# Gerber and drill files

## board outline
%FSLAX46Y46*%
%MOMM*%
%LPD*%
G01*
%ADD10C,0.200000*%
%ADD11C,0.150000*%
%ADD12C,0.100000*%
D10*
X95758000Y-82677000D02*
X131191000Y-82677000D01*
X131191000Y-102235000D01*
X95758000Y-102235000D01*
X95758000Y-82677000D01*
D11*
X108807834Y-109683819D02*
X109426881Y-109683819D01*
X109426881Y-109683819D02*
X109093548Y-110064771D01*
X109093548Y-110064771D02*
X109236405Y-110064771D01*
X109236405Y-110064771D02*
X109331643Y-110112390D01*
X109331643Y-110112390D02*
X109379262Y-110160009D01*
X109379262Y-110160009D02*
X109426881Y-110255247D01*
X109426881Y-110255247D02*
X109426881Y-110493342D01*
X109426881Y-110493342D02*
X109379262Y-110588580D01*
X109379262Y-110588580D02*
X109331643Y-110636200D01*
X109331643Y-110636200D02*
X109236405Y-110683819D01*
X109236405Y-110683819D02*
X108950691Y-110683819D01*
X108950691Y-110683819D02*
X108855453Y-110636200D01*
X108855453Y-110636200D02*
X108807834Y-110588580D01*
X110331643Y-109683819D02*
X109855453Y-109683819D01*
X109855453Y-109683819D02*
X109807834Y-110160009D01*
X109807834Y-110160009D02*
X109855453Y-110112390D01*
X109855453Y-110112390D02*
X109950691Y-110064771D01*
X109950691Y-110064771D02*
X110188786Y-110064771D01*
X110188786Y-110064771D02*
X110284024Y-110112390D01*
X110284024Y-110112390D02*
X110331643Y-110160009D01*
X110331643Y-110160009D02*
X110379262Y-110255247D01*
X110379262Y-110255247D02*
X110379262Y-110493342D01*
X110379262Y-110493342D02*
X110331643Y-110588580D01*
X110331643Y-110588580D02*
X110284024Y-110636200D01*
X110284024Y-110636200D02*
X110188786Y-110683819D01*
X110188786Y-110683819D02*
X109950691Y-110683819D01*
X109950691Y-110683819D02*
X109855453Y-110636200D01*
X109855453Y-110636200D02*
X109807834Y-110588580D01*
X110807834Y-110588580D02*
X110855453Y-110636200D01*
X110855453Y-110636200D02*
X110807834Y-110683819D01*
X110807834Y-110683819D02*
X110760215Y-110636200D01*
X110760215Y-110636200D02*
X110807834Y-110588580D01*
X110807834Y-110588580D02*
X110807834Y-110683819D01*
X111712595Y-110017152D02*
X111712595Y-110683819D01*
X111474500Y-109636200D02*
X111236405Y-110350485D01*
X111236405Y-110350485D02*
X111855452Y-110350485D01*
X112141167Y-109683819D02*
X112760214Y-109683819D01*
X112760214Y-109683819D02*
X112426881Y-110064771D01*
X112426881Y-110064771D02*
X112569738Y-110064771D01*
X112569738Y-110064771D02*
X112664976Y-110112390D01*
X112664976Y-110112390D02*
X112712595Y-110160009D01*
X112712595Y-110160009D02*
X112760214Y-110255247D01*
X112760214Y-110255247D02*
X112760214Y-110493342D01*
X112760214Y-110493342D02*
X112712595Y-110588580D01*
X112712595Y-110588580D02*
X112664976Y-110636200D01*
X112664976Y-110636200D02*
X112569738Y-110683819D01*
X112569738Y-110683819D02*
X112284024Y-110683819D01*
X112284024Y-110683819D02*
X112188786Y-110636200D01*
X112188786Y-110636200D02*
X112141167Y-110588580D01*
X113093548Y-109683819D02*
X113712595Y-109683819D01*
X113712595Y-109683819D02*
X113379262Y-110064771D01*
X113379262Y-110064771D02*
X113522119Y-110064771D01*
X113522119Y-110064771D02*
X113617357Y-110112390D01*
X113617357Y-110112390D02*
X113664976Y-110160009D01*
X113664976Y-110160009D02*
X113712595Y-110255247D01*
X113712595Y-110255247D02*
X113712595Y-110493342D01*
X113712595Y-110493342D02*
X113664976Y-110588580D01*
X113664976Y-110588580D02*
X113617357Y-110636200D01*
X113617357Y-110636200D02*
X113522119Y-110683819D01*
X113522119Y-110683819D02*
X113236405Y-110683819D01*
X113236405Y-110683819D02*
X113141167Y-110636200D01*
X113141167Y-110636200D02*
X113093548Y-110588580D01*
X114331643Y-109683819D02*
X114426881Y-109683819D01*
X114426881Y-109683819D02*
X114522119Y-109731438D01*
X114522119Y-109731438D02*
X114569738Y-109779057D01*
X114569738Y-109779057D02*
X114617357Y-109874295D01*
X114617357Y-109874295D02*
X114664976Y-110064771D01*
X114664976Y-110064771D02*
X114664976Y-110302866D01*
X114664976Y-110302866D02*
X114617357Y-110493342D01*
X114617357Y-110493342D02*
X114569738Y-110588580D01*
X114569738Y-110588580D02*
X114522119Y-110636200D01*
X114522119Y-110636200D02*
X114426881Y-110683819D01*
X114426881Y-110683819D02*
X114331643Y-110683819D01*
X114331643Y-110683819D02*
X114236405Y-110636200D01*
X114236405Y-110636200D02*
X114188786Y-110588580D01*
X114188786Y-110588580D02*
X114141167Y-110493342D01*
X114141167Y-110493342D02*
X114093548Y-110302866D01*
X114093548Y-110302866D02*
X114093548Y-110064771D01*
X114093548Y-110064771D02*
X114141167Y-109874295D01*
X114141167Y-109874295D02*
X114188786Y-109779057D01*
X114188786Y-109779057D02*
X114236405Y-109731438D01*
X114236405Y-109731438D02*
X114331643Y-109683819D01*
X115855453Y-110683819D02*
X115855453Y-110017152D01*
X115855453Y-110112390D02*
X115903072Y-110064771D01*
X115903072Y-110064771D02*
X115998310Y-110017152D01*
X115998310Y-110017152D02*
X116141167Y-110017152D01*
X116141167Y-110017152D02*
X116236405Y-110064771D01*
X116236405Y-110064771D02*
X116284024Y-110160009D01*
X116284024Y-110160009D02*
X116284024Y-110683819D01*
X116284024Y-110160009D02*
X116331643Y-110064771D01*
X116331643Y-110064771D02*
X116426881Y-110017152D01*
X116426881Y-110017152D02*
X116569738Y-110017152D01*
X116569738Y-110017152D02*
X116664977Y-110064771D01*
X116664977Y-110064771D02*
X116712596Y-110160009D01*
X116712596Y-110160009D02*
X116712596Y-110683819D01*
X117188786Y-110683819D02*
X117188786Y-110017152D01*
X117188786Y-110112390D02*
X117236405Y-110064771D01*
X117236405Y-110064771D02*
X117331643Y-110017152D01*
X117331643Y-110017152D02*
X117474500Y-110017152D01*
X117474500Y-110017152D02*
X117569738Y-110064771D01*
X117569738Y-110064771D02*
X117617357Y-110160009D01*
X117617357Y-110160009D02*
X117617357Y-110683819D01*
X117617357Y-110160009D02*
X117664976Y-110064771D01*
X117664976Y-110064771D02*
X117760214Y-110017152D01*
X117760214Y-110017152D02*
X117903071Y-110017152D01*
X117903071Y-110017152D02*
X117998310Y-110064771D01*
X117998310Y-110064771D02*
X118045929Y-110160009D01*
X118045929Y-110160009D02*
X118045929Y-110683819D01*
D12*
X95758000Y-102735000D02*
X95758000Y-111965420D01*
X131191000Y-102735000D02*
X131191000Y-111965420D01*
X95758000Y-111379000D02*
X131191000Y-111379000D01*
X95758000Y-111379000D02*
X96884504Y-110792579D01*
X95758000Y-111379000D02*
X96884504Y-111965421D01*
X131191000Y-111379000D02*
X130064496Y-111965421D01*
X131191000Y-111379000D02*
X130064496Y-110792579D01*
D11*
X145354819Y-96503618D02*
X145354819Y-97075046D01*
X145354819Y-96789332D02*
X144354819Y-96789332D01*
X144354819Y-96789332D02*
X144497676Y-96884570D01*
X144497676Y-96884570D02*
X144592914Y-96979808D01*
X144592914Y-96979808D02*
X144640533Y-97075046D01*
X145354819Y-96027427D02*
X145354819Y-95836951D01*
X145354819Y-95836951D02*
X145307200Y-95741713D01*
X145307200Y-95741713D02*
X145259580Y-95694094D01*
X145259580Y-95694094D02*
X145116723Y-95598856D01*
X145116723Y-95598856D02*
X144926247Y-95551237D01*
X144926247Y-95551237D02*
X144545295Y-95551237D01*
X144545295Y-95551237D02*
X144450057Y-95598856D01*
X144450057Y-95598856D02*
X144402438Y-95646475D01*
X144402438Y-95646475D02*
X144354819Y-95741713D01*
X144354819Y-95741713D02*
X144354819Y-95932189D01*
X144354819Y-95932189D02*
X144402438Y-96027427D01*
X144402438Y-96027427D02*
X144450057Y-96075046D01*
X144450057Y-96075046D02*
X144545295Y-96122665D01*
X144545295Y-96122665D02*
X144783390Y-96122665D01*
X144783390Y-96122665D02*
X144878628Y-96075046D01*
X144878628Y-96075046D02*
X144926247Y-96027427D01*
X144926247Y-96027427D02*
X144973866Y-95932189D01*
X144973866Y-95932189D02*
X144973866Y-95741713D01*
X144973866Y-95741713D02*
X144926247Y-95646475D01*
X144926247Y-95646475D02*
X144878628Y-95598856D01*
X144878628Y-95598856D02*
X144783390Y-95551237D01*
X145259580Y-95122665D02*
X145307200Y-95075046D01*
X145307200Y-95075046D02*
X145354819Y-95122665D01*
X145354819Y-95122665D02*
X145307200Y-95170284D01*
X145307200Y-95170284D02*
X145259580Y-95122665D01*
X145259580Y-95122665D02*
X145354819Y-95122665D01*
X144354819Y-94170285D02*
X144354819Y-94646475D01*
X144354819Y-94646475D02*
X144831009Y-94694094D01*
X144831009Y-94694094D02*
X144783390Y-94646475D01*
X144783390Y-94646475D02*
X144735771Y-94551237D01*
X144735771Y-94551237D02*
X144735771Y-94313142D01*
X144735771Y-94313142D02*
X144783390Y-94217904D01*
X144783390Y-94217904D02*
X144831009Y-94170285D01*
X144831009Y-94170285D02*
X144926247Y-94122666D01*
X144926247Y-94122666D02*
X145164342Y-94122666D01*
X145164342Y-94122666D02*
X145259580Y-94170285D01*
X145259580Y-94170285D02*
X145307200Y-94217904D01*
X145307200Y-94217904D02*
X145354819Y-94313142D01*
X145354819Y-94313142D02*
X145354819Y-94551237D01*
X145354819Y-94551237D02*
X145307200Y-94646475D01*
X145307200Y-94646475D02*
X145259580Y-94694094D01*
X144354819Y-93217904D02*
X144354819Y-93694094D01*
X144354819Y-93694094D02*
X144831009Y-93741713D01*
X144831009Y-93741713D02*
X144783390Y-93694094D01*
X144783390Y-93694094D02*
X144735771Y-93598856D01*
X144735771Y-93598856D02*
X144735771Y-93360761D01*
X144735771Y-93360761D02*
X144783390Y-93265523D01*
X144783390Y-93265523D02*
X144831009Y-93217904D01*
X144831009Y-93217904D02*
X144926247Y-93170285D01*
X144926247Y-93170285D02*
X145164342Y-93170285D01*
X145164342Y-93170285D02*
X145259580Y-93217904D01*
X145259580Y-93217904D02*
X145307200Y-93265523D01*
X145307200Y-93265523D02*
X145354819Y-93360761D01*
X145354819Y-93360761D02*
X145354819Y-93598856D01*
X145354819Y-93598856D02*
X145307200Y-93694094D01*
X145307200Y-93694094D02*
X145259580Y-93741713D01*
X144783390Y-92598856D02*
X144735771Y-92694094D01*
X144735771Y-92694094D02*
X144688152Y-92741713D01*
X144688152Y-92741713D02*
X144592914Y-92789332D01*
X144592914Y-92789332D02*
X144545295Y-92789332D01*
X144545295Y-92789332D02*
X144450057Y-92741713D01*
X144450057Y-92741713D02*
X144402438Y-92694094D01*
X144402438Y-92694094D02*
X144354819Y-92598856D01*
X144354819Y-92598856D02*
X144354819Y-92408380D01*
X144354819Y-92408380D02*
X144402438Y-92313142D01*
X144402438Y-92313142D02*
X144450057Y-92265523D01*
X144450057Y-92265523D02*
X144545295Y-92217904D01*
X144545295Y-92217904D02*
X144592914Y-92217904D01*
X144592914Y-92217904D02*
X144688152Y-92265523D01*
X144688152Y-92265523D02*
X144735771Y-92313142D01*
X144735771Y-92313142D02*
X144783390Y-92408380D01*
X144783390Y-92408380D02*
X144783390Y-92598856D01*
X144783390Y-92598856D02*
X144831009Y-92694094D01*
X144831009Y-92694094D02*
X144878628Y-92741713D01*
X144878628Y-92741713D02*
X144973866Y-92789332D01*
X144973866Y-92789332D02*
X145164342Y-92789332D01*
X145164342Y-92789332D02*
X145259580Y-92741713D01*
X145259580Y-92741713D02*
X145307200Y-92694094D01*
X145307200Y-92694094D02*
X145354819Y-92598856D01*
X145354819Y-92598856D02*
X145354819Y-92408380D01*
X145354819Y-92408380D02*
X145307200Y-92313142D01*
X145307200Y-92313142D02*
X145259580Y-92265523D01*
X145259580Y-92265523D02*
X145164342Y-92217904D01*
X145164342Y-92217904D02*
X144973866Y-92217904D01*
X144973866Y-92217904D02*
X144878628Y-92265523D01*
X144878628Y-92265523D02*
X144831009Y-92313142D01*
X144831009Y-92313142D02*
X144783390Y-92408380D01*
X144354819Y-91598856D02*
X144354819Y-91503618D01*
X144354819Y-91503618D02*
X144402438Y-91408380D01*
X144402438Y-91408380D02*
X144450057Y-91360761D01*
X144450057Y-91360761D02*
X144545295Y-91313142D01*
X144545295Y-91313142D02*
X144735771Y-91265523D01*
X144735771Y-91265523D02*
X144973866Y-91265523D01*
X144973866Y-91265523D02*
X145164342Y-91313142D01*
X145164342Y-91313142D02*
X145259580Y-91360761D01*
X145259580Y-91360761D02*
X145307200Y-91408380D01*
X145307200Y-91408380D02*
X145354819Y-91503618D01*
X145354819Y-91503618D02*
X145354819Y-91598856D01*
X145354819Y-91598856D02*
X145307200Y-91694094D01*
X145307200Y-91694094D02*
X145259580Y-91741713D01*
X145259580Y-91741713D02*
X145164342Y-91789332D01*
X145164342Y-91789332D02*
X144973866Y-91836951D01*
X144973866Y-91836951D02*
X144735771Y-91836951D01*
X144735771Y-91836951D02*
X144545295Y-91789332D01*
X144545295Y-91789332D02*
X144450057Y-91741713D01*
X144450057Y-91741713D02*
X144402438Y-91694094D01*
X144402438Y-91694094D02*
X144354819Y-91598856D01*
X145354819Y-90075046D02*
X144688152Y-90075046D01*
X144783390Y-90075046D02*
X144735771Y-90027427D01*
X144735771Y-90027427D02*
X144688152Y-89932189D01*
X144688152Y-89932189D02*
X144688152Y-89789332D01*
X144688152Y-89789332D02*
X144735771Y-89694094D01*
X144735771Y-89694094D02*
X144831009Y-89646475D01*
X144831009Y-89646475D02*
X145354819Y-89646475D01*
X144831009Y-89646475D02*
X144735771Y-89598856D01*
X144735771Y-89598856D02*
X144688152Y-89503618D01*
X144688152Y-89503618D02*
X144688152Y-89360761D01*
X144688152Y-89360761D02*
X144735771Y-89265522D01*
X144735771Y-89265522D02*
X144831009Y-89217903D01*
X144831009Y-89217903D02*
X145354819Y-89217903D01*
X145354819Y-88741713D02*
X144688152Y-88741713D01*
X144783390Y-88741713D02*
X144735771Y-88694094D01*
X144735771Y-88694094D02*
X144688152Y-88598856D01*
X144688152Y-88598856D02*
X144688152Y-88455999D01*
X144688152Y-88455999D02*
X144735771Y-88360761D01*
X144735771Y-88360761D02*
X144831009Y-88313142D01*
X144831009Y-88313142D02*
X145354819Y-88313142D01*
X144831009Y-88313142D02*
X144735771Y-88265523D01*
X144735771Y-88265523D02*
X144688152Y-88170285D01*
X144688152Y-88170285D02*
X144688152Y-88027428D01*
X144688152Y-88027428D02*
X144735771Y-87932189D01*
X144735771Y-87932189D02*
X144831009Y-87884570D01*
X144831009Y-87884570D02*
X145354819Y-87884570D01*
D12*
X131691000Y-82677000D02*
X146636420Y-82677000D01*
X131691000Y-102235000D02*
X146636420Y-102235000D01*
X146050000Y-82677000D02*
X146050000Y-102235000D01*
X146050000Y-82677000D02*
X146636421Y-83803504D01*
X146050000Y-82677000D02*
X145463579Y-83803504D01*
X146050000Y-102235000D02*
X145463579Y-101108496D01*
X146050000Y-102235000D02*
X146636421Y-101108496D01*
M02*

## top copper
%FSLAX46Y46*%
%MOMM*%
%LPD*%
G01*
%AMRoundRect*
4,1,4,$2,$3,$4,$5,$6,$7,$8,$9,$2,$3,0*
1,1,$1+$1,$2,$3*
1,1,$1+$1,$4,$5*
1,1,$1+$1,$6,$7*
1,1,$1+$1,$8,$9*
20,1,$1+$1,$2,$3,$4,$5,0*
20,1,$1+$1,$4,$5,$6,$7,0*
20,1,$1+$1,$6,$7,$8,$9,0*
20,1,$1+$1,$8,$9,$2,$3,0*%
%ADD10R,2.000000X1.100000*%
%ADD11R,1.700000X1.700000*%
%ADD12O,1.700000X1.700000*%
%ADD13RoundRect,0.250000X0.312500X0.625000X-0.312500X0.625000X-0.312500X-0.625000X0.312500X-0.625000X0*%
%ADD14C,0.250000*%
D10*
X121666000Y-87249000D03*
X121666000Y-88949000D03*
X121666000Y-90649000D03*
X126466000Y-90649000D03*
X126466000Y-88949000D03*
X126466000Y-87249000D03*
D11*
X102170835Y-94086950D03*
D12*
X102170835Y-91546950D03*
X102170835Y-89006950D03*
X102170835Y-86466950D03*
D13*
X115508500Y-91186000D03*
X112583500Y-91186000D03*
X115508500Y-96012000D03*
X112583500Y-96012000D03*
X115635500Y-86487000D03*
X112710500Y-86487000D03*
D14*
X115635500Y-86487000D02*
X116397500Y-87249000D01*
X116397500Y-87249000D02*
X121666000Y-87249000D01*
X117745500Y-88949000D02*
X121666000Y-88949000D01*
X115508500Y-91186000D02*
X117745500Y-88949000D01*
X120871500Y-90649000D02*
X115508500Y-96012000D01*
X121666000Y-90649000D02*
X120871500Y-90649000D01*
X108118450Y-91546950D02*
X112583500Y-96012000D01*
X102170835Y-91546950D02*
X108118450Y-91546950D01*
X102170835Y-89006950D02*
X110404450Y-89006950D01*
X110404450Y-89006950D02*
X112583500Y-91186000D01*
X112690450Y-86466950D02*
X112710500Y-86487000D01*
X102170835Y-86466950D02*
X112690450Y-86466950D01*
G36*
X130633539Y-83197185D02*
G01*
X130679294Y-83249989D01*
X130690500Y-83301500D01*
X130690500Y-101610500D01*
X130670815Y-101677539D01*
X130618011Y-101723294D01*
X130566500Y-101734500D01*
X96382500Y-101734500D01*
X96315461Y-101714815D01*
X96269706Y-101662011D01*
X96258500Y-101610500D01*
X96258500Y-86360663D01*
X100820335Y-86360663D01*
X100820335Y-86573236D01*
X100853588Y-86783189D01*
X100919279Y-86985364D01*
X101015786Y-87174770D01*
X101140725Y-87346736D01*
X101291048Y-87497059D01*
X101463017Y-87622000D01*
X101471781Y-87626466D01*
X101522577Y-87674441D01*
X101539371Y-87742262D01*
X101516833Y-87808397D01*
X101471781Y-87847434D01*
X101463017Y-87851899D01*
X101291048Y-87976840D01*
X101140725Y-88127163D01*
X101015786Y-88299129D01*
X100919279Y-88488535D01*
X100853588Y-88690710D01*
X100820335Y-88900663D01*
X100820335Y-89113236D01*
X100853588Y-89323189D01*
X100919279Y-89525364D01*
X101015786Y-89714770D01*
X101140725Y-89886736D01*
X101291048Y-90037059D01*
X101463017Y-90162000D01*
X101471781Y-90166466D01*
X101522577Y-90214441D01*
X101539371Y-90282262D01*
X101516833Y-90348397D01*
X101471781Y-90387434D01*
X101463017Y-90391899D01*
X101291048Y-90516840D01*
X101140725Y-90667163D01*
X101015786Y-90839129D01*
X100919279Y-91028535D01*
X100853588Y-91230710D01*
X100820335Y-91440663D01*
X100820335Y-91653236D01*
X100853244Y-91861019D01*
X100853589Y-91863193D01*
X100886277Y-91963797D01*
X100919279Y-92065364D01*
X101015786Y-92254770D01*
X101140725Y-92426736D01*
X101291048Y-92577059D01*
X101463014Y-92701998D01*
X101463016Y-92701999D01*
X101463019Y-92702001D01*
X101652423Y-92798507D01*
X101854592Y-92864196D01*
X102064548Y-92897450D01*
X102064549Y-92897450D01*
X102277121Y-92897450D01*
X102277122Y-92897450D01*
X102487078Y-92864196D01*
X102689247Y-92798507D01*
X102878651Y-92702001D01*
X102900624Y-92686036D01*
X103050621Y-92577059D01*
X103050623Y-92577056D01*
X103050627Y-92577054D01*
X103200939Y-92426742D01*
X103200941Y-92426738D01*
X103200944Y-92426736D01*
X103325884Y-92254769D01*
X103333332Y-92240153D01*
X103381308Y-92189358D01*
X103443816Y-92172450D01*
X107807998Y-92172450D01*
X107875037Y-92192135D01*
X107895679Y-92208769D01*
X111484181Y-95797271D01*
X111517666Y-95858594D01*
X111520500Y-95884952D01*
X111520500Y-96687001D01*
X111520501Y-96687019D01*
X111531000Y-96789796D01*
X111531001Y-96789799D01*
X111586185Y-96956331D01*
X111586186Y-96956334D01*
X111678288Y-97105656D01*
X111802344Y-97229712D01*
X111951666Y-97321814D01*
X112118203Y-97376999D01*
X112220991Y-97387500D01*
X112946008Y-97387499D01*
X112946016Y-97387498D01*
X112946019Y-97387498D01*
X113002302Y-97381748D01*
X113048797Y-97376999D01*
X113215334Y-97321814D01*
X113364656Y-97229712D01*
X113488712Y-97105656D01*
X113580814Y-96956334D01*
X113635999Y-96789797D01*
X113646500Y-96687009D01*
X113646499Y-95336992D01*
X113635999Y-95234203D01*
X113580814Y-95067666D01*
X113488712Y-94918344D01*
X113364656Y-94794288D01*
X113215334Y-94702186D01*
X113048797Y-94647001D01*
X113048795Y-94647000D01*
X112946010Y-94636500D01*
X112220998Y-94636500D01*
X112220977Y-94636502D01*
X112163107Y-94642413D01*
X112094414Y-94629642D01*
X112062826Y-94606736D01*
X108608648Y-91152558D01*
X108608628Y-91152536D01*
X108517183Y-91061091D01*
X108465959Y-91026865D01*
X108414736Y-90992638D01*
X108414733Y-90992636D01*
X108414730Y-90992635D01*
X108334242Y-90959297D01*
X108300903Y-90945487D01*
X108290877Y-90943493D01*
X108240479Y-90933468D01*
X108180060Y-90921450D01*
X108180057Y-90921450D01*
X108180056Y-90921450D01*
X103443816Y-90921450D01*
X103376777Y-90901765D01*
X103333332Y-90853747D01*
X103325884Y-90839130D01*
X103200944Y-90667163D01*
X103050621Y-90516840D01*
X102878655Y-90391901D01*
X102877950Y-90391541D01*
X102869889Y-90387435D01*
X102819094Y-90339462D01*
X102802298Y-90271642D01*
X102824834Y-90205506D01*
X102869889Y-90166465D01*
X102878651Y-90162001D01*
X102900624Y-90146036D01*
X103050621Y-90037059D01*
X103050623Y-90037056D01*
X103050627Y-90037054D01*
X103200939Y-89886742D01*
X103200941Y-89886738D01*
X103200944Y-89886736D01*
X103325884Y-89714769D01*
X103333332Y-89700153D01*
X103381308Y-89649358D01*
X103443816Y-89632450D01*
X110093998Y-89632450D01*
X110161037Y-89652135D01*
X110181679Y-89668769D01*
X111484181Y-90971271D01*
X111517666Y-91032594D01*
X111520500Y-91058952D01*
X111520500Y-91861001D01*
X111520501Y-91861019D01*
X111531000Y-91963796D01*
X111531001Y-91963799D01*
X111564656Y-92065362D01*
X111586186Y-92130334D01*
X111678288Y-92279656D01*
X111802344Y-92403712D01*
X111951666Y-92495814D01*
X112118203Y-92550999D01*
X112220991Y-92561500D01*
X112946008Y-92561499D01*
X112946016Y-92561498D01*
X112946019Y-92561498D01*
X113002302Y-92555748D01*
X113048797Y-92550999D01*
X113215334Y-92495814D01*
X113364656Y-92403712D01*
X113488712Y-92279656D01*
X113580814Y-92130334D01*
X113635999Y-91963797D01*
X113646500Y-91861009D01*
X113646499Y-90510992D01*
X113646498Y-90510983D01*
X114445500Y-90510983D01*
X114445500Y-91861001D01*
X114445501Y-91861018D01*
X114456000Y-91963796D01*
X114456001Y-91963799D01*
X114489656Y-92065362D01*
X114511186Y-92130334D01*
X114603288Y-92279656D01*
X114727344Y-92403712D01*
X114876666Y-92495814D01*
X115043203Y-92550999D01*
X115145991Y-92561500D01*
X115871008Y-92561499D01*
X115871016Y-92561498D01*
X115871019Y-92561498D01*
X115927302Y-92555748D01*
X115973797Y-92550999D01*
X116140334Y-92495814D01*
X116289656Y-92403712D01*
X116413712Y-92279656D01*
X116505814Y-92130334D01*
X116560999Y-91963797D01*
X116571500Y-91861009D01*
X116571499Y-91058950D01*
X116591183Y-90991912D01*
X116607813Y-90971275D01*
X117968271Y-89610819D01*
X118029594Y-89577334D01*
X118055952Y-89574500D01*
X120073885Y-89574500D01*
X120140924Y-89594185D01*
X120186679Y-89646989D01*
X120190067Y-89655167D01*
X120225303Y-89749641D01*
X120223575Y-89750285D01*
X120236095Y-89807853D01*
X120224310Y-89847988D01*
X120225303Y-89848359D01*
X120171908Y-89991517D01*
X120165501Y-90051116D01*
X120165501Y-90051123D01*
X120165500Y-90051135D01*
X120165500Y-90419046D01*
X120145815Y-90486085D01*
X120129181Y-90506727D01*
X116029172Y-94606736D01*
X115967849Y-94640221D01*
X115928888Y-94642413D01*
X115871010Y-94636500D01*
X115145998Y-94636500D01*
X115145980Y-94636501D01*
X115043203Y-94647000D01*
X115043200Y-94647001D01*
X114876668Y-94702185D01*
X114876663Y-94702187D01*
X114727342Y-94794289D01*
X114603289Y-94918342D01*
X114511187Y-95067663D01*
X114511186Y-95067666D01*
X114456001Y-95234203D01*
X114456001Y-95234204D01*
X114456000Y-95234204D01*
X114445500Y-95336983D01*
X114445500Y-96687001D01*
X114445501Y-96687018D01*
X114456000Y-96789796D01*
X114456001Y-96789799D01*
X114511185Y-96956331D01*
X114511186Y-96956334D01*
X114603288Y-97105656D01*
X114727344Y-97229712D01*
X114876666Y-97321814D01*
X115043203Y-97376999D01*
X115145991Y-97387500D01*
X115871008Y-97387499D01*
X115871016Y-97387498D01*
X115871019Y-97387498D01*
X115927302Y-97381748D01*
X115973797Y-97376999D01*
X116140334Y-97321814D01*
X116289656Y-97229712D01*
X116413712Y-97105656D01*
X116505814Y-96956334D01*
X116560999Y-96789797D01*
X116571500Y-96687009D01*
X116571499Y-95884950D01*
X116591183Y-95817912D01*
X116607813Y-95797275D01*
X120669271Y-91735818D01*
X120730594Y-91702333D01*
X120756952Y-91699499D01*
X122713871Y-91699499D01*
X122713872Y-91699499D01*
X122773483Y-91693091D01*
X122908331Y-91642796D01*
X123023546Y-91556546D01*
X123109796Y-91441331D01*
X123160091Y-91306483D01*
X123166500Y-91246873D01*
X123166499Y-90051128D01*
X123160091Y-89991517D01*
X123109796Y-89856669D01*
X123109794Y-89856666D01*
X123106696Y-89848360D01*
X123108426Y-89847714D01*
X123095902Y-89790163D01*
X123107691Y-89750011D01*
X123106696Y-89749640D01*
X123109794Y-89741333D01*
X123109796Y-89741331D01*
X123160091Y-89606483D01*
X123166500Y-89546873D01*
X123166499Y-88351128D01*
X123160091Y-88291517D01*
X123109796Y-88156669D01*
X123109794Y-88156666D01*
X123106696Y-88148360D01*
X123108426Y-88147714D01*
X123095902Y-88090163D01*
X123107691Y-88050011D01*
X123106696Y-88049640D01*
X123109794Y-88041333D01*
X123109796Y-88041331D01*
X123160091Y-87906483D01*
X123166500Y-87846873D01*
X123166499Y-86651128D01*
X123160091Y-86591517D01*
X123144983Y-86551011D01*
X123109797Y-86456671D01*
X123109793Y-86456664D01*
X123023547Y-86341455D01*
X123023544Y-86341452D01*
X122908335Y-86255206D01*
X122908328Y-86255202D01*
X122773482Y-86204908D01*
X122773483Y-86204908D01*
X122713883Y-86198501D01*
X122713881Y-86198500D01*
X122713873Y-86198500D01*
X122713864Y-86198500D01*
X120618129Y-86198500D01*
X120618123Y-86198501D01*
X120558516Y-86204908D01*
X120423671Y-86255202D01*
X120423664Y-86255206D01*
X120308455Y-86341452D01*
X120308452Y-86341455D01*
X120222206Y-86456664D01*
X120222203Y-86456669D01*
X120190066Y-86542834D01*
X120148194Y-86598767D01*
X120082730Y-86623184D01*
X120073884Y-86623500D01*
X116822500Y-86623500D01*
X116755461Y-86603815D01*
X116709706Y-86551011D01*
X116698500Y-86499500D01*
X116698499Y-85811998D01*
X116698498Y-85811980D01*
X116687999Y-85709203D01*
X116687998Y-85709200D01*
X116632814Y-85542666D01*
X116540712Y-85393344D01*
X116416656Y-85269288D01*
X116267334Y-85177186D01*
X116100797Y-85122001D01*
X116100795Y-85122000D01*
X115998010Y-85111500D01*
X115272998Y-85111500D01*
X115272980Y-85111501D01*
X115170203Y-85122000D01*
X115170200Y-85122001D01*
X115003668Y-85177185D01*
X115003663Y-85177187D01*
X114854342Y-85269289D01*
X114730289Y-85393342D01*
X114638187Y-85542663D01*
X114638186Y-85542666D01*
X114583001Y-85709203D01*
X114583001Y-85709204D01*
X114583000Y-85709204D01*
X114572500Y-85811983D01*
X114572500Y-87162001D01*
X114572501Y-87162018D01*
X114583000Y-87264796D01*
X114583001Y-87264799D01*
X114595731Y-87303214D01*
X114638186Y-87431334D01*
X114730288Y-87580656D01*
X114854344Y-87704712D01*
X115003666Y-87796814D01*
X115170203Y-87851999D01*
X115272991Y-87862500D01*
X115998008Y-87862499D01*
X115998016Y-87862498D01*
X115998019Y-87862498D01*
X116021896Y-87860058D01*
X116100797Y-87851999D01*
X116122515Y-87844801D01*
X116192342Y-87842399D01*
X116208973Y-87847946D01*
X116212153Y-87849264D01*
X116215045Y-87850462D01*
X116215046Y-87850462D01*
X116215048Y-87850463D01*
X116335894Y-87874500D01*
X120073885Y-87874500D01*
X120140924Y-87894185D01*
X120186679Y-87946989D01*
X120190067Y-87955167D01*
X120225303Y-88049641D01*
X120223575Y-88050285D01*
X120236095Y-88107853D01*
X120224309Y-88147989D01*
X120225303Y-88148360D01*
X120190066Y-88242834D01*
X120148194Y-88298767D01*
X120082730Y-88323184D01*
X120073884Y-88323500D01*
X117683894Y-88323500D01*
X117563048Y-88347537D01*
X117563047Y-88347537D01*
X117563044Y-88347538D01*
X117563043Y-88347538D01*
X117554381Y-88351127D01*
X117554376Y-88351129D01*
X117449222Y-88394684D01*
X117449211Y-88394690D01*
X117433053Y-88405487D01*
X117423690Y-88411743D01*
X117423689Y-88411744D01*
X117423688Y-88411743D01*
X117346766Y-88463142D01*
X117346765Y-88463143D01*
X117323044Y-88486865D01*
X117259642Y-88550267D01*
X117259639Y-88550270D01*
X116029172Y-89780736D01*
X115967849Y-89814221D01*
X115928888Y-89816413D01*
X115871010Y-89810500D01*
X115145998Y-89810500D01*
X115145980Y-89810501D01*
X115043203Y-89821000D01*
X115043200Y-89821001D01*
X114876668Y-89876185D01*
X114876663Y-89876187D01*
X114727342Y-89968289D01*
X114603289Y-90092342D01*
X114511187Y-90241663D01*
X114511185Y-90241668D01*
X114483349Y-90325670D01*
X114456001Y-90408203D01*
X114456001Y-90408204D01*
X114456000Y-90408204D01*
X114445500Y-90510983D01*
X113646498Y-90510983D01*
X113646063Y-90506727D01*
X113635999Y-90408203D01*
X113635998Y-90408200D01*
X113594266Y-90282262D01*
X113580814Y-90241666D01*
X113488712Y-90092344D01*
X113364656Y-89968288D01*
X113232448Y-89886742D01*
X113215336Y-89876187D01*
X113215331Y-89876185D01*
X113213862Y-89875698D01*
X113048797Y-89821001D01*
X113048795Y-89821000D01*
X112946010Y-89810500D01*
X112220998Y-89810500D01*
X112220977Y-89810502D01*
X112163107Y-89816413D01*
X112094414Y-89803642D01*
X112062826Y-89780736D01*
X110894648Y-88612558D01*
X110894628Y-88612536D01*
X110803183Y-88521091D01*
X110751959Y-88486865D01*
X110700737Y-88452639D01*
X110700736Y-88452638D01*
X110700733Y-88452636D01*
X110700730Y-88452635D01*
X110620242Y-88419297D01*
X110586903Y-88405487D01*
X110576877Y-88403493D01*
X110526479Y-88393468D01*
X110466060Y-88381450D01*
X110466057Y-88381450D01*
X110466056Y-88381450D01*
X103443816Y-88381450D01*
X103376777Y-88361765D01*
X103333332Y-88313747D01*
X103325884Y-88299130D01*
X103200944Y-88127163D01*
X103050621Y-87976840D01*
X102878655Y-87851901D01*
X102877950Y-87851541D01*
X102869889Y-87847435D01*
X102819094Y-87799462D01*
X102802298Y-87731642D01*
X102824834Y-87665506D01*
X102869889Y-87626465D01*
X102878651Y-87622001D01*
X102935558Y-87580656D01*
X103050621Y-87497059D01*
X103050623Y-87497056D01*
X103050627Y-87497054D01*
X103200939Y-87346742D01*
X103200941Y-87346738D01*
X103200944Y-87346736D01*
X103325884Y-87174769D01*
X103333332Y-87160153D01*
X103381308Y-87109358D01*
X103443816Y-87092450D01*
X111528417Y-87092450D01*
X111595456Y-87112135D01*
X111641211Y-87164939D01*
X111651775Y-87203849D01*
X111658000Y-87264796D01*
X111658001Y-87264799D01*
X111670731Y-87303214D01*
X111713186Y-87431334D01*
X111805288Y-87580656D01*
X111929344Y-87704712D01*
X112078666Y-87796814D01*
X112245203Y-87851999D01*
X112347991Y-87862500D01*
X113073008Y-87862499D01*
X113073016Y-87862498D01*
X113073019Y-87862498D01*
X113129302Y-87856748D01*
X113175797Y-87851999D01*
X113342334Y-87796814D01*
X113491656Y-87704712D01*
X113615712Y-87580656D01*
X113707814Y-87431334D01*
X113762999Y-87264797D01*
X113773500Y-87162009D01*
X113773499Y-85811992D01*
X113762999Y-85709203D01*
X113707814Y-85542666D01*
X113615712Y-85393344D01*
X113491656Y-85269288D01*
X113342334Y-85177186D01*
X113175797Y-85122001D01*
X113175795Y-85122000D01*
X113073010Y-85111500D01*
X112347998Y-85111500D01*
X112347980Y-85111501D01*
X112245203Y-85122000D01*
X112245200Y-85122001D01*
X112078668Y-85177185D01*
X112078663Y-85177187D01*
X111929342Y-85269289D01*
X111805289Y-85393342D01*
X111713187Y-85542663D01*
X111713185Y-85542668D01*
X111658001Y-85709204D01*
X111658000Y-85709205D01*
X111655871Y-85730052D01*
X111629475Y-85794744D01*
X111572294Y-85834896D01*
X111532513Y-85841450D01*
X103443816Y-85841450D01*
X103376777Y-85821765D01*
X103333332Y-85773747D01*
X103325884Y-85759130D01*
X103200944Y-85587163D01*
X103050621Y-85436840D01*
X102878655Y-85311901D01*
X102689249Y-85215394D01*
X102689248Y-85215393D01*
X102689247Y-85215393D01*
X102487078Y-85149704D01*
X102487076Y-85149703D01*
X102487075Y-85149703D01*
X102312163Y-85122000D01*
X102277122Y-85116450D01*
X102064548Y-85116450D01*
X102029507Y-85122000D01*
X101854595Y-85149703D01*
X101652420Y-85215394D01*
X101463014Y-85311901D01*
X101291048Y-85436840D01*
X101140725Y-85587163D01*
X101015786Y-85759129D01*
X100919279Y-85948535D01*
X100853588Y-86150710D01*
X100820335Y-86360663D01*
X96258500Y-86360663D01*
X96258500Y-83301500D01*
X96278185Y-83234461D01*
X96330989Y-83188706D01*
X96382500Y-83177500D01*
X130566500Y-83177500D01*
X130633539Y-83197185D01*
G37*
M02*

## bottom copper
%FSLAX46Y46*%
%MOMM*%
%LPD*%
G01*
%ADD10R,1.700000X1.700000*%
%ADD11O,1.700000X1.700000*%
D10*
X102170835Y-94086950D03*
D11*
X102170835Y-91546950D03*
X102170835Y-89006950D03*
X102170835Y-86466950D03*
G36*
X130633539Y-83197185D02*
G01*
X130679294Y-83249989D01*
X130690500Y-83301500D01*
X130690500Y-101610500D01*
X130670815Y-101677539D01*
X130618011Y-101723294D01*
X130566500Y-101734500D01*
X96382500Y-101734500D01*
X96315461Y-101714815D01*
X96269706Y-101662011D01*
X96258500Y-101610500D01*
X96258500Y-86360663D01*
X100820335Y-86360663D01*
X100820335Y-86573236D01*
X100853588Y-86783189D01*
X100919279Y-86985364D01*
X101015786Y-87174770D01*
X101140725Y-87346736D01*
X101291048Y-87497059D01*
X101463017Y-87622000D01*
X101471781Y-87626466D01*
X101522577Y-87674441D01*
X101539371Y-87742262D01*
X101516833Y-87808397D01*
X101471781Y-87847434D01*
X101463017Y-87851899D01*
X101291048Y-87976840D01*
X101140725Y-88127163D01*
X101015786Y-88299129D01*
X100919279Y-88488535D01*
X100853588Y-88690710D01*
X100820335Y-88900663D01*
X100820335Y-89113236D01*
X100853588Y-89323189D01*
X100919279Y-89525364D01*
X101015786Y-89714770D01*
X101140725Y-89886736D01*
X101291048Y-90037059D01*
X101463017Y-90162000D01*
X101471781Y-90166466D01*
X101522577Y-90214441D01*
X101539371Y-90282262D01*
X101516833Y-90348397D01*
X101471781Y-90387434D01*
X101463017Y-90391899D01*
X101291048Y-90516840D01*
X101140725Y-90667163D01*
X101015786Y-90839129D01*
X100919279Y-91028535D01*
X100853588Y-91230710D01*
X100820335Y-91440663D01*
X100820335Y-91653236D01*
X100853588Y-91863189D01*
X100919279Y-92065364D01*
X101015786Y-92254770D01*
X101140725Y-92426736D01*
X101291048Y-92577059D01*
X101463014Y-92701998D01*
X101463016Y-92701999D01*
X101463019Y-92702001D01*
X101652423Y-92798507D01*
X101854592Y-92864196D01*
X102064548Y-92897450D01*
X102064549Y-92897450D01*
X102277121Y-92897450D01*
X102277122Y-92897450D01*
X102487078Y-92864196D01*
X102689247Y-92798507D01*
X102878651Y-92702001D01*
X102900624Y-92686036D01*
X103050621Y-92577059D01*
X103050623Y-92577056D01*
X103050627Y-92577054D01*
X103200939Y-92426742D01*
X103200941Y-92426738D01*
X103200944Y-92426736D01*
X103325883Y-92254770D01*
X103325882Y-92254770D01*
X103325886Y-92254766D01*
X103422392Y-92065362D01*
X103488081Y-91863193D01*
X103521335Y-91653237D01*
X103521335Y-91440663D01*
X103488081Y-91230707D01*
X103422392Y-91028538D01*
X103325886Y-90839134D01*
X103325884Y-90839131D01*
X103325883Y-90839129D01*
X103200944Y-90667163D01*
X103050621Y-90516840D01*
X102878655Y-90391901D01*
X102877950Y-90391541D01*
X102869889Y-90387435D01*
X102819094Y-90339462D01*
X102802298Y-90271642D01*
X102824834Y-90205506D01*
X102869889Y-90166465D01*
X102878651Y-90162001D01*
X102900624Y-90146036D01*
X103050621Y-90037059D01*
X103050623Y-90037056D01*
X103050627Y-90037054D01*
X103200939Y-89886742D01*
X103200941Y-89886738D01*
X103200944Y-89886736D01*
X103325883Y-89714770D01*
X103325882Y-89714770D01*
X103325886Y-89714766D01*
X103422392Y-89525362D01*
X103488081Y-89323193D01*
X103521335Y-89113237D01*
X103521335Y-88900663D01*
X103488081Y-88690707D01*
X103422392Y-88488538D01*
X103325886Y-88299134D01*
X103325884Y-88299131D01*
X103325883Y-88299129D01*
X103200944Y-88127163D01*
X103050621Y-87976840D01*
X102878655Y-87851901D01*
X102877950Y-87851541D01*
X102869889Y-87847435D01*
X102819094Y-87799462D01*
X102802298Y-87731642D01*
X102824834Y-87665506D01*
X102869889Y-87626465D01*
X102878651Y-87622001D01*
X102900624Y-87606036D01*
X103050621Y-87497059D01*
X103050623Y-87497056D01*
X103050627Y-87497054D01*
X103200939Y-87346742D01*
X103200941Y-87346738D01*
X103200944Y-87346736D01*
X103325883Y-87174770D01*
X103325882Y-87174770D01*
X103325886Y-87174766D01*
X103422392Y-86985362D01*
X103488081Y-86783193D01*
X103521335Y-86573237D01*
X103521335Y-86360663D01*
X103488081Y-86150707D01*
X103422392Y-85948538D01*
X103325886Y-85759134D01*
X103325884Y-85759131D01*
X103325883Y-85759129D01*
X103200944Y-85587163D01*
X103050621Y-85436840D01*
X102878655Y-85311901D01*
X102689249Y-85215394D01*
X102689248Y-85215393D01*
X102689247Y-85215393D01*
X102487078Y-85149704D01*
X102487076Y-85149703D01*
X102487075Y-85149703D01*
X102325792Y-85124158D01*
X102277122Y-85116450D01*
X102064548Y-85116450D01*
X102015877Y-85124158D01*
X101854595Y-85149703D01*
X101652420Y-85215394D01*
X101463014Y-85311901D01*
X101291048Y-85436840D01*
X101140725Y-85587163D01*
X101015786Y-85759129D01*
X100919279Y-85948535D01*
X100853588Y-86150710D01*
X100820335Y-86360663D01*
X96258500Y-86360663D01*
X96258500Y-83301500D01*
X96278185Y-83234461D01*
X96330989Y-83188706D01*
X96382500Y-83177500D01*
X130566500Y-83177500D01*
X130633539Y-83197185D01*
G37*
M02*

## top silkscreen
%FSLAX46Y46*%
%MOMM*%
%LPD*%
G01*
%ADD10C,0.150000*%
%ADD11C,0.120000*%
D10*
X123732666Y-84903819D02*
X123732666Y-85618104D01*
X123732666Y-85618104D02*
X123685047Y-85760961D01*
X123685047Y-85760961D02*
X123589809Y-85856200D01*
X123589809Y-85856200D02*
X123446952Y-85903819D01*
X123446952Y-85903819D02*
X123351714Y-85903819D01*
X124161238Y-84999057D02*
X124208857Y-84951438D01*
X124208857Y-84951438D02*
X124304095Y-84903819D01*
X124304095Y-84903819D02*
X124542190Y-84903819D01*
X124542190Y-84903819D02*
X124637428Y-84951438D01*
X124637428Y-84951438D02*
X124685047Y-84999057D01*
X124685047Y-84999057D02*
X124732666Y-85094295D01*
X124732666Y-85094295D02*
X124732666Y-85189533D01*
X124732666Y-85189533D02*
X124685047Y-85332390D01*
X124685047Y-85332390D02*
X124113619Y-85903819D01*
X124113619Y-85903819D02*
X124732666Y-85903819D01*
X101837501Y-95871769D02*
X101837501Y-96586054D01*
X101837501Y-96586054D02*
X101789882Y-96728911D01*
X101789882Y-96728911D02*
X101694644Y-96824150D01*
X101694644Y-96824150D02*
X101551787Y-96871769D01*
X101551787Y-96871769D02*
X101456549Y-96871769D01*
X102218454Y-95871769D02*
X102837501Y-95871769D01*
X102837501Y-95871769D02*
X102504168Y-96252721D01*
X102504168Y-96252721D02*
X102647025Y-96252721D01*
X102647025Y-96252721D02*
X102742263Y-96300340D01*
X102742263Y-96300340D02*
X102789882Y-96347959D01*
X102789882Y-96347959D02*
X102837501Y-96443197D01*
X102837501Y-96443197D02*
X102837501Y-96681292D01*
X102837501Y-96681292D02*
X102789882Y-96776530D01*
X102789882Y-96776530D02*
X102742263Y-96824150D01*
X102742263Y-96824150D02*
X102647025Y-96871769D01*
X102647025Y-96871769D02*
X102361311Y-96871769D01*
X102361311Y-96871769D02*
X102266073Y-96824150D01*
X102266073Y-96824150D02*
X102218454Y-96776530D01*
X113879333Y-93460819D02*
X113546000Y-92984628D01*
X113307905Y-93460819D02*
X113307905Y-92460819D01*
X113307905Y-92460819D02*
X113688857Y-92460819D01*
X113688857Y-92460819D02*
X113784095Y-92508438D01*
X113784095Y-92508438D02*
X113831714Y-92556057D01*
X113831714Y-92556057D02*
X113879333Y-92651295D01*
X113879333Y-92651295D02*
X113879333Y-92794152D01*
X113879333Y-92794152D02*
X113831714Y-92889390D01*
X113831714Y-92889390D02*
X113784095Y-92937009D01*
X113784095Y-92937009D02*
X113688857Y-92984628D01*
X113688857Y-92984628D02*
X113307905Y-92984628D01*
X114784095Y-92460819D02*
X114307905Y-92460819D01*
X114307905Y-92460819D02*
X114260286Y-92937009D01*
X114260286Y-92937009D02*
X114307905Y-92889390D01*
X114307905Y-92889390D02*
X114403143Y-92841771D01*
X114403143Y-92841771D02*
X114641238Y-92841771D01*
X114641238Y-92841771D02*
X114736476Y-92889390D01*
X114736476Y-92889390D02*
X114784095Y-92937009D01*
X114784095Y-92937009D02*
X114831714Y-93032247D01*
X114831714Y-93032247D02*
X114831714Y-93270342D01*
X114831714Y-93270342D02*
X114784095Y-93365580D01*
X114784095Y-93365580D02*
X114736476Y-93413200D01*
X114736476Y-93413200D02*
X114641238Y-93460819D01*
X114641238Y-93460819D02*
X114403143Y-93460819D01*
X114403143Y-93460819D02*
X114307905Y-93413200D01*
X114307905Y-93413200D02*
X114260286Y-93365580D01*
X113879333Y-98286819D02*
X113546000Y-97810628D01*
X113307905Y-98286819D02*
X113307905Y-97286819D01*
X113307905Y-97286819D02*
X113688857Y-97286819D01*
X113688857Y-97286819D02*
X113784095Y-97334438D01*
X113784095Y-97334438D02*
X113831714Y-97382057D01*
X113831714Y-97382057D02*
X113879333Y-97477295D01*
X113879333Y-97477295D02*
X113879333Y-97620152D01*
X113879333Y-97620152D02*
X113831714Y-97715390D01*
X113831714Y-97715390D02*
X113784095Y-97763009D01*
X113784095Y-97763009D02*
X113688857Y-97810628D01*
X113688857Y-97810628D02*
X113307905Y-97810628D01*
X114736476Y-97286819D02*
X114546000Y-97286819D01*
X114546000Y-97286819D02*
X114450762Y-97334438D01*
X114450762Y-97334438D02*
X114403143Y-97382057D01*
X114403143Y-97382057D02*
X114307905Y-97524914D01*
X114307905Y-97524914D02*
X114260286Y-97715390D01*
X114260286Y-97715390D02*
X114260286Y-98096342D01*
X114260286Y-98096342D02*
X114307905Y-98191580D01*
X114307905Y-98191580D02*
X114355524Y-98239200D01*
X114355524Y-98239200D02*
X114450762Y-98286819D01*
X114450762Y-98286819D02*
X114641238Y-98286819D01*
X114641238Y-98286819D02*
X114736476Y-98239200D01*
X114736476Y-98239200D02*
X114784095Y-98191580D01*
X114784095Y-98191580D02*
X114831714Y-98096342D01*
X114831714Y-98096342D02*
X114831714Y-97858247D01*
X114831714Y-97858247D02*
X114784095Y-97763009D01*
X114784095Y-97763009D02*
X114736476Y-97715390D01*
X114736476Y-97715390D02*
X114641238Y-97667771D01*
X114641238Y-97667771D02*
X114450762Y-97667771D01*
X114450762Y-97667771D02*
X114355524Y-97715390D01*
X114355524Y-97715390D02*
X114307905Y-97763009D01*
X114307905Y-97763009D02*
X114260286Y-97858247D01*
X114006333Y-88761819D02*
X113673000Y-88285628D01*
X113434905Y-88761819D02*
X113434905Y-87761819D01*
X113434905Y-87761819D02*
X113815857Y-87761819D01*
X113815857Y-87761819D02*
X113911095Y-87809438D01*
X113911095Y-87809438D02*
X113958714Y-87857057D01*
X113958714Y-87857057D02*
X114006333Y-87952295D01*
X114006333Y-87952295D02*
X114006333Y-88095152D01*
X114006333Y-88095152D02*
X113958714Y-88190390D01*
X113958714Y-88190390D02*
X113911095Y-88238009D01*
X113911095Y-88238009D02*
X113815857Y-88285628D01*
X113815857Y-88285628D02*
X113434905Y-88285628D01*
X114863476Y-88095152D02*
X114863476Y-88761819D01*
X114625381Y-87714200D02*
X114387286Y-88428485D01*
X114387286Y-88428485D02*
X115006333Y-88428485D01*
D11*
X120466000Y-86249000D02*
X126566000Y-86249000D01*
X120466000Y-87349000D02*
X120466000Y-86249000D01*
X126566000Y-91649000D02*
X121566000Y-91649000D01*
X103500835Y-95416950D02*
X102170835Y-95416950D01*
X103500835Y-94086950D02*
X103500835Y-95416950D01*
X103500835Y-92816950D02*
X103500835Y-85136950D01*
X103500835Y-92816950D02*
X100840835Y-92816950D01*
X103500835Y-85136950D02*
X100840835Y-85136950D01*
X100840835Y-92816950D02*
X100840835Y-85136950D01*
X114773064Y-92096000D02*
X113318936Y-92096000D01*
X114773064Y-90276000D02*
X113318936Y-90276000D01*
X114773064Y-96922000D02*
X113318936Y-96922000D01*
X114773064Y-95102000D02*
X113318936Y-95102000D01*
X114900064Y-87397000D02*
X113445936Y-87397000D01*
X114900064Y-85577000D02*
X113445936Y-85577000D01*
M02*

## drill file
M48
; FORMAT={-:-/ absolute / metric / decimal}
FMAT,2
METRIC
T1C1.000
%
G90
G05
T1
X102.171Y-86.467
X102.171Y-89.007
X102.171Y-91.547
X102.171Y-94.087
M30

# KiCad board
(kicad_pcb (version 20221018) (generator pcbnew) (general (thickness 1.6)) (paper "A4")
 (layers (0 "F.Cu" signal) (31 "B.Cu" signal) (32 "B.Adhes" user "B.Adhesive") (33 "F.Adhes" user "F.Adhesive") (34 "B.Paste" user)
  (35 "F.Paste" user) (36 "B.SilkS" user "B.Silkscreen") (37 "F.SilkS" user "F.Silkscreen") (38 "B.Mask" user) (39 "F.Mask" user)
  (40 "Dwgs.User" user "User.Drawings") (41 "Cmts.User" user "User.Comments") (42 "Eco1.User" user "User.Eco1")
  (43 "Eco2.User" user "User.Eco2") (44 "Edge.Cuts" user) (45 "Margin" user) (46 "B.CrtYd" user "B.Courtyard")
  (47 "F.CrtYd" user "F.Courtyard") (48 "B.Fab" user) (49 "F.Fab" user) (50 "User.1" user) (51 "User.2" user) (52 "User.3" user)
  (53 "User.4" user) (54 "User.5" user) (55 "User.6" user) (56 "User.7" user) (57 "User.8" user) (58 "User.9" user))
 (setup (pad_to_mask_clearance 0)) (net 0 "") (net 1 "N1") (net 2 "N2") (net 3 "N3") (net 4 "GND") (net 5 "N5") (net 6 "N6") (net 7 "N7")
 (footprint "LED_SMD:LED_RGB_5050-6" (layer "F.Cu") (at 124.066 88.949)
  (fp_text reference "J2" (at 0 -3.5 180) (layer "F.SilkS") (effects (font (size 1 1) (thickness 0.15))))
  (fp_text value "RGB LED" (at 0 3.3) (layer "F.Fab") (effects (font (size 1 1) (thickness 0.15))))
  (fp_line (start -3.6 -2.7) (end 2.5 -2.7) (stroke (width 0.12) (type solid)) (layer "F.SilkS"))
  (fp_line (start -3.6 -1.6) (end -3.6 -2.7) (stroke (width 0.12) (type solid)) (layer "F.SilkS"))
  (fp_line (start 2.5 2.7) (end -2.5 2.7) (stroke (width 0.12) (type solid)) (layer "F.SilkS"))
  (pad "1" smd rect (at -2.4 -1.7 90) (size 1.1 2) (layers "F.Cu" "F.Paste" "F.Mask") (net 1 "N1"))
  (pad "2" smd rect (at -2.4 0 90) (size 1.1 2) (layers "F.Cu" "F.Paste" "F.Mask") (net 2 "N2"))
  (pad "3" smd rect (at -2.4 1.7 90) (size 1.1 2) (layers "F.Cu" "F.Paste" "F.Mask") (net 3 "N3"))
  (pad "4" smd rect (at 2.4 1.7 90) (size 1.1 2) (layers "F.Cu" "F.Paste" "F.Mask") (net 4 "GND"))
  (pad "5" smd rect (at 2.4 0 90) (size 1.1 2) (layers "F.Cu" "F.Paste" "F.Mask") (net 4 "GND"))
  (pad "6" smd rect (at 2.4 -1.7 90) (size 1.1 2) (layers "F.Cu" "F.Paste" "F.Mask") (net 4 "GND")))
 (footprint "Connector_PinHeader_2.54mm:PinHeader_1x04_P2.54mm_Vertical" (layer "F.Cu") (at 102.170835 94.08695 180)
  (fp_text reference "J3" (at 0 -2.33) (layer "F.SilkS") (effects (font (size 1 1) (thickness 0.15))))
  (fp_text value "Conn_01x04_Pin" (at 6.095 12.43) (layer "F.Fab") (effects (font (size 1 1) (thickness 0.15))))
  (fp_line (start -1.33 -1.33) (end 0 -1.33) (stroke (width 0.12) (type solid)) (layer "F.SilkS"))
  (fp_line (start -1.33 0) (end -1.33 -1.33) (stroke (width 0.12) (type solid)) (layer "F.SilkS"))
  (fp_line (start -1.33 1.27) (end -1.33 8.95) (stroke (width 0.12) (type solid)) (layer "F.SilkS"))
  (fp_line (start -1.33 1.27) (end 1.33 1.27) (stroke (width 0.12) (type solid)) (layer "F.SilkS"))
  (fp_line (start -1.33 8.95) (end 1.33 8.95) (stroke (width 0.12) (type solid)) (layer "F.SilkS"))
  (fp_line (start 1.33 1.27) (end 1.33 8.95) (stroke (width 0.12) (type solid)) (layer "F.SilkS"))
  (pad "1" thru_hole rect (at 0 0 180) (size 1.7 1.7) (drill 1) (layers "*.Cu" "*.Mask") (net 4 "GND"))
  (pad "2" thru_hole oval (at 0 2.54 180) (size 1.7 1.7) (drill 1) (layers "*.Cu" "*.Mask") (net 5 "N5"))
  (pad "3" thru_hole oval (at 0 5.08 180) (size 1.7 1.7) (drill 1) (layers "*.Cu" "*.Mask") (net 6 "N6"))
  (pad "4" thru_hole oval (at 0 7.62 180) (size 1.7 1.7) (drill 1) (layers "*.Cu" "*.Mask") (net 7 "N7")))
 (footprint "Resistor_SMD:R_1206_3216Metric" (layer "F.Cu") (at 114.046 91.186 180)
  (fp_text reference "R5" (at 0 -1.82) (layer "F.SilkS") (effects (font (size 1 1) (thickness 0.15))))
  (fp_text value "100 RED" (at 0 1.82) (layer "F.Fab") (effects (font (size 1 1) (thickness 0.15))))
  (fp_line (start -0.727064 -0.91) (end 0.727064 -0.91) (stroke (width 0.12) (type solid)) (layer "F.SilkS"))
  (fp_line (start -0.727064 0.91) (end 0.727064 0.91) (stroke (width 0.12) (type solid)) (layer "F.SilkS"))
  (pad "1" smd roundrect (at -1.4625 0 180) (size 1.125 1.75) (layers "F.Cu" "F.Paste" "F.Mask") (roundrect_rratio 0.222222) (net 2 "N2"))
  (pad "2" smd roundrect (at 1.4625 0 180) (size 1.125 1.75) (layers "F.Cu" "F.Paste" "F.Mask") (roundrect_rratio 0.222222) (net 6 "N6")))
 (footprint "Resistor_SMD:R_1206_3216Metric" (layer "F.Cu") (at 114.046 96.012 180)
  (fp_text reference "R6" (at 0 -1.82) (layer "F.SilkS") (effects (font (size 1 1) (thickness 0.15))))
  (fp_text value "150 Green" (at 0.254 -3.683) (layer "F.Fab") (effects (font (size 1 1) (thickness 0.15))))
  (fp_line (start -0.727064 -0.91) (end 0.727064 -0.91) (stroke (width 0.12) (type solid)) (layer "F.SilkS"))
  (fp_line (start -0.727064 0.91) (end 0.727064 0.91) (stroke (width 0.12) (type solid)) (layer "F.SilkS"))
  (pad "1" smd roundrect (at -1.4625 0 180) (size 1.125 1.75) (layers "F.Cu" "F.Paste" "F.Mask") (roundrect_rratio 0.222222) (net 3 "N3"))
  (pad "2" smd roundrect (at 1.4625 0 180) (size 1.125 1.75) (layers "F.Cu" "F.Paste" "F.Mask") (roundrect_rratio 0.222222) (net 5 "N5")))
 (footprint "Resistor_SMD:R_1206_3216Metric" (layer "F.Cu") (at 114.173 86.487 180)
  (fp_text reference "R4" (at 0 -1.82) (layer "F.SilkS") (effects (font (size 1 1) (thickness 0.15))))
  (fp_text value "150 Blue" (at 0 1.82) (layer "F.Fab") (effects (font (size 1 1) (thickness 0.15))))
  (fp_line (start -0.727064 -0.91) (end 0.727064 -0.91) (stroke (width 0.12) (type solid)) (layer "F.SilkS"))
  (fp_line (start -0.727064 0.91) (end 0.727064 0.91) (stroke (width 0.12) (type solid)) (layer "F.SilkS"))
  (pad "1" smd roundrect (at -1.4625 0 180) (size 1.125 1.75) (layers "F.Cu" "F.Paste" "F.Mask") (roundrect_rratio 0.222222) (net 1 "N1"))
  (pad "2" smd roundrect (at 1.4625 0 180) (size 1.125 1.75) (layers "F.Cu" "F.Paste" "F.Mask") (roundrect_rratio 0.222222) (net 7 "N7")))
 (gr_rect (start 95.758 82.677) (end 131.191 102.235) (stroke (width 0.2) (type default)) (fill none) (layer "Edge.Cuts"))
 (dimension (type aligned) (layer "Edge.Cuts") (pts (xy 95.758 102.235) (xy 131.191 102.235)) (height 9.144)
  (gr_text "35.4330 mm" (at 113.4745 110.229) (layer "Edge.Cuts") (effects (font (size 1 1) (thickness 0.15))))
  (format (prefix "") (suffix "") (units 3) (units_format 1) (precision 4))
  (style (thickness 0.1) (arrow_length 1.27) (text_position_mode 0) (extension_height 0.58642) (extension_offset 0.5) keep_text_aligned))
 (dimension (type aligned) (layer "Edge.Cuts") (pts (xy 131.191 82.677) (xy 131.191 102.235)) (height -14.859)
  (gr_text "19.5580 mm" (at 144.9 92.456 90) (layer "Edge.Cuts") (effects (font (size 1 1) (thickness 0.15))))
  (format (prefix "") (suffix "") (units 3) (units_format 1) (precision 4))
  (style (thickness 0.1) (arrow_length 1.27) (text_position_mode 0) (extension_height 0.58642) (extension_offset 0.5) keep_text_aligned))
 (segment (start 115.6355 86.487) (end 116.3975 87.249) (width 0.25) (layer "F.Cu") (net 1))
 (segment (start 116.3975 87.249) (end 121.666 87.249) (width 0.25) (layer "F.Cu") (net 1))
 (segment (start 117.7455 88.949) (end 121.666 88.949) (width 0.25) (layer "F.Cu") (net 2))
 (segment (start 115.5085 91.186) (end 117.7455 88.949) (width 0.25) (layer "F.Cu") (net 2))
 (segment (start 120.8715 90.649) (end 115.5085 96.012) (width 0.25) (layer "F.Cu") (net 3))
 (segment (start 121.666 90.649) (end 120.8715 90.649) (width 0.25) (layer "F.Cu") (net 3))
 (segment (start 108.11845 91.54695) (end 112.5835 96.012) (width 0.25) (layer "F.Cu") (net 5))
 (segment (start 102.170835 91.54695) (end 108.11845 91.54695) (width 0.25) (layer "F.Cu") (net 5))
 (segment (start 102.170835 89.00695) (end 110.40445 89.00695) (width 0.25) (layer "F.Cu") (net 6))
 (segment (start 110.40445 89.00695) (end 112.5835 91.186) (width 0.25) (layer "F.Cu") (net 6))
 (segment (start 112.69045 86.46695) (end 112.7105 86.487) (width 0.25) (layer "F.Cu") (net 7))
 (segment (start 102.170835 86.46695) (end 112.69045 86.46695) (width 0.25) (layer "F.Cu") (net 7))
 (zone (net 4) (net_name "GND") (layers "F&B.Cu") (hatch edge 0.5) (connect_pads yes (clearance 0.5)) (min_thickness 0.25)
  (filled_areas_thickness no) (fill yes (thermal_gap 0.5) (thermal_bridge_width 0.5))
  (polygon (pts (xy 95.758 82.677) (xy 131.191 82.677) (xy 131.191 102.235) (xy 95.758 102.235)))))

